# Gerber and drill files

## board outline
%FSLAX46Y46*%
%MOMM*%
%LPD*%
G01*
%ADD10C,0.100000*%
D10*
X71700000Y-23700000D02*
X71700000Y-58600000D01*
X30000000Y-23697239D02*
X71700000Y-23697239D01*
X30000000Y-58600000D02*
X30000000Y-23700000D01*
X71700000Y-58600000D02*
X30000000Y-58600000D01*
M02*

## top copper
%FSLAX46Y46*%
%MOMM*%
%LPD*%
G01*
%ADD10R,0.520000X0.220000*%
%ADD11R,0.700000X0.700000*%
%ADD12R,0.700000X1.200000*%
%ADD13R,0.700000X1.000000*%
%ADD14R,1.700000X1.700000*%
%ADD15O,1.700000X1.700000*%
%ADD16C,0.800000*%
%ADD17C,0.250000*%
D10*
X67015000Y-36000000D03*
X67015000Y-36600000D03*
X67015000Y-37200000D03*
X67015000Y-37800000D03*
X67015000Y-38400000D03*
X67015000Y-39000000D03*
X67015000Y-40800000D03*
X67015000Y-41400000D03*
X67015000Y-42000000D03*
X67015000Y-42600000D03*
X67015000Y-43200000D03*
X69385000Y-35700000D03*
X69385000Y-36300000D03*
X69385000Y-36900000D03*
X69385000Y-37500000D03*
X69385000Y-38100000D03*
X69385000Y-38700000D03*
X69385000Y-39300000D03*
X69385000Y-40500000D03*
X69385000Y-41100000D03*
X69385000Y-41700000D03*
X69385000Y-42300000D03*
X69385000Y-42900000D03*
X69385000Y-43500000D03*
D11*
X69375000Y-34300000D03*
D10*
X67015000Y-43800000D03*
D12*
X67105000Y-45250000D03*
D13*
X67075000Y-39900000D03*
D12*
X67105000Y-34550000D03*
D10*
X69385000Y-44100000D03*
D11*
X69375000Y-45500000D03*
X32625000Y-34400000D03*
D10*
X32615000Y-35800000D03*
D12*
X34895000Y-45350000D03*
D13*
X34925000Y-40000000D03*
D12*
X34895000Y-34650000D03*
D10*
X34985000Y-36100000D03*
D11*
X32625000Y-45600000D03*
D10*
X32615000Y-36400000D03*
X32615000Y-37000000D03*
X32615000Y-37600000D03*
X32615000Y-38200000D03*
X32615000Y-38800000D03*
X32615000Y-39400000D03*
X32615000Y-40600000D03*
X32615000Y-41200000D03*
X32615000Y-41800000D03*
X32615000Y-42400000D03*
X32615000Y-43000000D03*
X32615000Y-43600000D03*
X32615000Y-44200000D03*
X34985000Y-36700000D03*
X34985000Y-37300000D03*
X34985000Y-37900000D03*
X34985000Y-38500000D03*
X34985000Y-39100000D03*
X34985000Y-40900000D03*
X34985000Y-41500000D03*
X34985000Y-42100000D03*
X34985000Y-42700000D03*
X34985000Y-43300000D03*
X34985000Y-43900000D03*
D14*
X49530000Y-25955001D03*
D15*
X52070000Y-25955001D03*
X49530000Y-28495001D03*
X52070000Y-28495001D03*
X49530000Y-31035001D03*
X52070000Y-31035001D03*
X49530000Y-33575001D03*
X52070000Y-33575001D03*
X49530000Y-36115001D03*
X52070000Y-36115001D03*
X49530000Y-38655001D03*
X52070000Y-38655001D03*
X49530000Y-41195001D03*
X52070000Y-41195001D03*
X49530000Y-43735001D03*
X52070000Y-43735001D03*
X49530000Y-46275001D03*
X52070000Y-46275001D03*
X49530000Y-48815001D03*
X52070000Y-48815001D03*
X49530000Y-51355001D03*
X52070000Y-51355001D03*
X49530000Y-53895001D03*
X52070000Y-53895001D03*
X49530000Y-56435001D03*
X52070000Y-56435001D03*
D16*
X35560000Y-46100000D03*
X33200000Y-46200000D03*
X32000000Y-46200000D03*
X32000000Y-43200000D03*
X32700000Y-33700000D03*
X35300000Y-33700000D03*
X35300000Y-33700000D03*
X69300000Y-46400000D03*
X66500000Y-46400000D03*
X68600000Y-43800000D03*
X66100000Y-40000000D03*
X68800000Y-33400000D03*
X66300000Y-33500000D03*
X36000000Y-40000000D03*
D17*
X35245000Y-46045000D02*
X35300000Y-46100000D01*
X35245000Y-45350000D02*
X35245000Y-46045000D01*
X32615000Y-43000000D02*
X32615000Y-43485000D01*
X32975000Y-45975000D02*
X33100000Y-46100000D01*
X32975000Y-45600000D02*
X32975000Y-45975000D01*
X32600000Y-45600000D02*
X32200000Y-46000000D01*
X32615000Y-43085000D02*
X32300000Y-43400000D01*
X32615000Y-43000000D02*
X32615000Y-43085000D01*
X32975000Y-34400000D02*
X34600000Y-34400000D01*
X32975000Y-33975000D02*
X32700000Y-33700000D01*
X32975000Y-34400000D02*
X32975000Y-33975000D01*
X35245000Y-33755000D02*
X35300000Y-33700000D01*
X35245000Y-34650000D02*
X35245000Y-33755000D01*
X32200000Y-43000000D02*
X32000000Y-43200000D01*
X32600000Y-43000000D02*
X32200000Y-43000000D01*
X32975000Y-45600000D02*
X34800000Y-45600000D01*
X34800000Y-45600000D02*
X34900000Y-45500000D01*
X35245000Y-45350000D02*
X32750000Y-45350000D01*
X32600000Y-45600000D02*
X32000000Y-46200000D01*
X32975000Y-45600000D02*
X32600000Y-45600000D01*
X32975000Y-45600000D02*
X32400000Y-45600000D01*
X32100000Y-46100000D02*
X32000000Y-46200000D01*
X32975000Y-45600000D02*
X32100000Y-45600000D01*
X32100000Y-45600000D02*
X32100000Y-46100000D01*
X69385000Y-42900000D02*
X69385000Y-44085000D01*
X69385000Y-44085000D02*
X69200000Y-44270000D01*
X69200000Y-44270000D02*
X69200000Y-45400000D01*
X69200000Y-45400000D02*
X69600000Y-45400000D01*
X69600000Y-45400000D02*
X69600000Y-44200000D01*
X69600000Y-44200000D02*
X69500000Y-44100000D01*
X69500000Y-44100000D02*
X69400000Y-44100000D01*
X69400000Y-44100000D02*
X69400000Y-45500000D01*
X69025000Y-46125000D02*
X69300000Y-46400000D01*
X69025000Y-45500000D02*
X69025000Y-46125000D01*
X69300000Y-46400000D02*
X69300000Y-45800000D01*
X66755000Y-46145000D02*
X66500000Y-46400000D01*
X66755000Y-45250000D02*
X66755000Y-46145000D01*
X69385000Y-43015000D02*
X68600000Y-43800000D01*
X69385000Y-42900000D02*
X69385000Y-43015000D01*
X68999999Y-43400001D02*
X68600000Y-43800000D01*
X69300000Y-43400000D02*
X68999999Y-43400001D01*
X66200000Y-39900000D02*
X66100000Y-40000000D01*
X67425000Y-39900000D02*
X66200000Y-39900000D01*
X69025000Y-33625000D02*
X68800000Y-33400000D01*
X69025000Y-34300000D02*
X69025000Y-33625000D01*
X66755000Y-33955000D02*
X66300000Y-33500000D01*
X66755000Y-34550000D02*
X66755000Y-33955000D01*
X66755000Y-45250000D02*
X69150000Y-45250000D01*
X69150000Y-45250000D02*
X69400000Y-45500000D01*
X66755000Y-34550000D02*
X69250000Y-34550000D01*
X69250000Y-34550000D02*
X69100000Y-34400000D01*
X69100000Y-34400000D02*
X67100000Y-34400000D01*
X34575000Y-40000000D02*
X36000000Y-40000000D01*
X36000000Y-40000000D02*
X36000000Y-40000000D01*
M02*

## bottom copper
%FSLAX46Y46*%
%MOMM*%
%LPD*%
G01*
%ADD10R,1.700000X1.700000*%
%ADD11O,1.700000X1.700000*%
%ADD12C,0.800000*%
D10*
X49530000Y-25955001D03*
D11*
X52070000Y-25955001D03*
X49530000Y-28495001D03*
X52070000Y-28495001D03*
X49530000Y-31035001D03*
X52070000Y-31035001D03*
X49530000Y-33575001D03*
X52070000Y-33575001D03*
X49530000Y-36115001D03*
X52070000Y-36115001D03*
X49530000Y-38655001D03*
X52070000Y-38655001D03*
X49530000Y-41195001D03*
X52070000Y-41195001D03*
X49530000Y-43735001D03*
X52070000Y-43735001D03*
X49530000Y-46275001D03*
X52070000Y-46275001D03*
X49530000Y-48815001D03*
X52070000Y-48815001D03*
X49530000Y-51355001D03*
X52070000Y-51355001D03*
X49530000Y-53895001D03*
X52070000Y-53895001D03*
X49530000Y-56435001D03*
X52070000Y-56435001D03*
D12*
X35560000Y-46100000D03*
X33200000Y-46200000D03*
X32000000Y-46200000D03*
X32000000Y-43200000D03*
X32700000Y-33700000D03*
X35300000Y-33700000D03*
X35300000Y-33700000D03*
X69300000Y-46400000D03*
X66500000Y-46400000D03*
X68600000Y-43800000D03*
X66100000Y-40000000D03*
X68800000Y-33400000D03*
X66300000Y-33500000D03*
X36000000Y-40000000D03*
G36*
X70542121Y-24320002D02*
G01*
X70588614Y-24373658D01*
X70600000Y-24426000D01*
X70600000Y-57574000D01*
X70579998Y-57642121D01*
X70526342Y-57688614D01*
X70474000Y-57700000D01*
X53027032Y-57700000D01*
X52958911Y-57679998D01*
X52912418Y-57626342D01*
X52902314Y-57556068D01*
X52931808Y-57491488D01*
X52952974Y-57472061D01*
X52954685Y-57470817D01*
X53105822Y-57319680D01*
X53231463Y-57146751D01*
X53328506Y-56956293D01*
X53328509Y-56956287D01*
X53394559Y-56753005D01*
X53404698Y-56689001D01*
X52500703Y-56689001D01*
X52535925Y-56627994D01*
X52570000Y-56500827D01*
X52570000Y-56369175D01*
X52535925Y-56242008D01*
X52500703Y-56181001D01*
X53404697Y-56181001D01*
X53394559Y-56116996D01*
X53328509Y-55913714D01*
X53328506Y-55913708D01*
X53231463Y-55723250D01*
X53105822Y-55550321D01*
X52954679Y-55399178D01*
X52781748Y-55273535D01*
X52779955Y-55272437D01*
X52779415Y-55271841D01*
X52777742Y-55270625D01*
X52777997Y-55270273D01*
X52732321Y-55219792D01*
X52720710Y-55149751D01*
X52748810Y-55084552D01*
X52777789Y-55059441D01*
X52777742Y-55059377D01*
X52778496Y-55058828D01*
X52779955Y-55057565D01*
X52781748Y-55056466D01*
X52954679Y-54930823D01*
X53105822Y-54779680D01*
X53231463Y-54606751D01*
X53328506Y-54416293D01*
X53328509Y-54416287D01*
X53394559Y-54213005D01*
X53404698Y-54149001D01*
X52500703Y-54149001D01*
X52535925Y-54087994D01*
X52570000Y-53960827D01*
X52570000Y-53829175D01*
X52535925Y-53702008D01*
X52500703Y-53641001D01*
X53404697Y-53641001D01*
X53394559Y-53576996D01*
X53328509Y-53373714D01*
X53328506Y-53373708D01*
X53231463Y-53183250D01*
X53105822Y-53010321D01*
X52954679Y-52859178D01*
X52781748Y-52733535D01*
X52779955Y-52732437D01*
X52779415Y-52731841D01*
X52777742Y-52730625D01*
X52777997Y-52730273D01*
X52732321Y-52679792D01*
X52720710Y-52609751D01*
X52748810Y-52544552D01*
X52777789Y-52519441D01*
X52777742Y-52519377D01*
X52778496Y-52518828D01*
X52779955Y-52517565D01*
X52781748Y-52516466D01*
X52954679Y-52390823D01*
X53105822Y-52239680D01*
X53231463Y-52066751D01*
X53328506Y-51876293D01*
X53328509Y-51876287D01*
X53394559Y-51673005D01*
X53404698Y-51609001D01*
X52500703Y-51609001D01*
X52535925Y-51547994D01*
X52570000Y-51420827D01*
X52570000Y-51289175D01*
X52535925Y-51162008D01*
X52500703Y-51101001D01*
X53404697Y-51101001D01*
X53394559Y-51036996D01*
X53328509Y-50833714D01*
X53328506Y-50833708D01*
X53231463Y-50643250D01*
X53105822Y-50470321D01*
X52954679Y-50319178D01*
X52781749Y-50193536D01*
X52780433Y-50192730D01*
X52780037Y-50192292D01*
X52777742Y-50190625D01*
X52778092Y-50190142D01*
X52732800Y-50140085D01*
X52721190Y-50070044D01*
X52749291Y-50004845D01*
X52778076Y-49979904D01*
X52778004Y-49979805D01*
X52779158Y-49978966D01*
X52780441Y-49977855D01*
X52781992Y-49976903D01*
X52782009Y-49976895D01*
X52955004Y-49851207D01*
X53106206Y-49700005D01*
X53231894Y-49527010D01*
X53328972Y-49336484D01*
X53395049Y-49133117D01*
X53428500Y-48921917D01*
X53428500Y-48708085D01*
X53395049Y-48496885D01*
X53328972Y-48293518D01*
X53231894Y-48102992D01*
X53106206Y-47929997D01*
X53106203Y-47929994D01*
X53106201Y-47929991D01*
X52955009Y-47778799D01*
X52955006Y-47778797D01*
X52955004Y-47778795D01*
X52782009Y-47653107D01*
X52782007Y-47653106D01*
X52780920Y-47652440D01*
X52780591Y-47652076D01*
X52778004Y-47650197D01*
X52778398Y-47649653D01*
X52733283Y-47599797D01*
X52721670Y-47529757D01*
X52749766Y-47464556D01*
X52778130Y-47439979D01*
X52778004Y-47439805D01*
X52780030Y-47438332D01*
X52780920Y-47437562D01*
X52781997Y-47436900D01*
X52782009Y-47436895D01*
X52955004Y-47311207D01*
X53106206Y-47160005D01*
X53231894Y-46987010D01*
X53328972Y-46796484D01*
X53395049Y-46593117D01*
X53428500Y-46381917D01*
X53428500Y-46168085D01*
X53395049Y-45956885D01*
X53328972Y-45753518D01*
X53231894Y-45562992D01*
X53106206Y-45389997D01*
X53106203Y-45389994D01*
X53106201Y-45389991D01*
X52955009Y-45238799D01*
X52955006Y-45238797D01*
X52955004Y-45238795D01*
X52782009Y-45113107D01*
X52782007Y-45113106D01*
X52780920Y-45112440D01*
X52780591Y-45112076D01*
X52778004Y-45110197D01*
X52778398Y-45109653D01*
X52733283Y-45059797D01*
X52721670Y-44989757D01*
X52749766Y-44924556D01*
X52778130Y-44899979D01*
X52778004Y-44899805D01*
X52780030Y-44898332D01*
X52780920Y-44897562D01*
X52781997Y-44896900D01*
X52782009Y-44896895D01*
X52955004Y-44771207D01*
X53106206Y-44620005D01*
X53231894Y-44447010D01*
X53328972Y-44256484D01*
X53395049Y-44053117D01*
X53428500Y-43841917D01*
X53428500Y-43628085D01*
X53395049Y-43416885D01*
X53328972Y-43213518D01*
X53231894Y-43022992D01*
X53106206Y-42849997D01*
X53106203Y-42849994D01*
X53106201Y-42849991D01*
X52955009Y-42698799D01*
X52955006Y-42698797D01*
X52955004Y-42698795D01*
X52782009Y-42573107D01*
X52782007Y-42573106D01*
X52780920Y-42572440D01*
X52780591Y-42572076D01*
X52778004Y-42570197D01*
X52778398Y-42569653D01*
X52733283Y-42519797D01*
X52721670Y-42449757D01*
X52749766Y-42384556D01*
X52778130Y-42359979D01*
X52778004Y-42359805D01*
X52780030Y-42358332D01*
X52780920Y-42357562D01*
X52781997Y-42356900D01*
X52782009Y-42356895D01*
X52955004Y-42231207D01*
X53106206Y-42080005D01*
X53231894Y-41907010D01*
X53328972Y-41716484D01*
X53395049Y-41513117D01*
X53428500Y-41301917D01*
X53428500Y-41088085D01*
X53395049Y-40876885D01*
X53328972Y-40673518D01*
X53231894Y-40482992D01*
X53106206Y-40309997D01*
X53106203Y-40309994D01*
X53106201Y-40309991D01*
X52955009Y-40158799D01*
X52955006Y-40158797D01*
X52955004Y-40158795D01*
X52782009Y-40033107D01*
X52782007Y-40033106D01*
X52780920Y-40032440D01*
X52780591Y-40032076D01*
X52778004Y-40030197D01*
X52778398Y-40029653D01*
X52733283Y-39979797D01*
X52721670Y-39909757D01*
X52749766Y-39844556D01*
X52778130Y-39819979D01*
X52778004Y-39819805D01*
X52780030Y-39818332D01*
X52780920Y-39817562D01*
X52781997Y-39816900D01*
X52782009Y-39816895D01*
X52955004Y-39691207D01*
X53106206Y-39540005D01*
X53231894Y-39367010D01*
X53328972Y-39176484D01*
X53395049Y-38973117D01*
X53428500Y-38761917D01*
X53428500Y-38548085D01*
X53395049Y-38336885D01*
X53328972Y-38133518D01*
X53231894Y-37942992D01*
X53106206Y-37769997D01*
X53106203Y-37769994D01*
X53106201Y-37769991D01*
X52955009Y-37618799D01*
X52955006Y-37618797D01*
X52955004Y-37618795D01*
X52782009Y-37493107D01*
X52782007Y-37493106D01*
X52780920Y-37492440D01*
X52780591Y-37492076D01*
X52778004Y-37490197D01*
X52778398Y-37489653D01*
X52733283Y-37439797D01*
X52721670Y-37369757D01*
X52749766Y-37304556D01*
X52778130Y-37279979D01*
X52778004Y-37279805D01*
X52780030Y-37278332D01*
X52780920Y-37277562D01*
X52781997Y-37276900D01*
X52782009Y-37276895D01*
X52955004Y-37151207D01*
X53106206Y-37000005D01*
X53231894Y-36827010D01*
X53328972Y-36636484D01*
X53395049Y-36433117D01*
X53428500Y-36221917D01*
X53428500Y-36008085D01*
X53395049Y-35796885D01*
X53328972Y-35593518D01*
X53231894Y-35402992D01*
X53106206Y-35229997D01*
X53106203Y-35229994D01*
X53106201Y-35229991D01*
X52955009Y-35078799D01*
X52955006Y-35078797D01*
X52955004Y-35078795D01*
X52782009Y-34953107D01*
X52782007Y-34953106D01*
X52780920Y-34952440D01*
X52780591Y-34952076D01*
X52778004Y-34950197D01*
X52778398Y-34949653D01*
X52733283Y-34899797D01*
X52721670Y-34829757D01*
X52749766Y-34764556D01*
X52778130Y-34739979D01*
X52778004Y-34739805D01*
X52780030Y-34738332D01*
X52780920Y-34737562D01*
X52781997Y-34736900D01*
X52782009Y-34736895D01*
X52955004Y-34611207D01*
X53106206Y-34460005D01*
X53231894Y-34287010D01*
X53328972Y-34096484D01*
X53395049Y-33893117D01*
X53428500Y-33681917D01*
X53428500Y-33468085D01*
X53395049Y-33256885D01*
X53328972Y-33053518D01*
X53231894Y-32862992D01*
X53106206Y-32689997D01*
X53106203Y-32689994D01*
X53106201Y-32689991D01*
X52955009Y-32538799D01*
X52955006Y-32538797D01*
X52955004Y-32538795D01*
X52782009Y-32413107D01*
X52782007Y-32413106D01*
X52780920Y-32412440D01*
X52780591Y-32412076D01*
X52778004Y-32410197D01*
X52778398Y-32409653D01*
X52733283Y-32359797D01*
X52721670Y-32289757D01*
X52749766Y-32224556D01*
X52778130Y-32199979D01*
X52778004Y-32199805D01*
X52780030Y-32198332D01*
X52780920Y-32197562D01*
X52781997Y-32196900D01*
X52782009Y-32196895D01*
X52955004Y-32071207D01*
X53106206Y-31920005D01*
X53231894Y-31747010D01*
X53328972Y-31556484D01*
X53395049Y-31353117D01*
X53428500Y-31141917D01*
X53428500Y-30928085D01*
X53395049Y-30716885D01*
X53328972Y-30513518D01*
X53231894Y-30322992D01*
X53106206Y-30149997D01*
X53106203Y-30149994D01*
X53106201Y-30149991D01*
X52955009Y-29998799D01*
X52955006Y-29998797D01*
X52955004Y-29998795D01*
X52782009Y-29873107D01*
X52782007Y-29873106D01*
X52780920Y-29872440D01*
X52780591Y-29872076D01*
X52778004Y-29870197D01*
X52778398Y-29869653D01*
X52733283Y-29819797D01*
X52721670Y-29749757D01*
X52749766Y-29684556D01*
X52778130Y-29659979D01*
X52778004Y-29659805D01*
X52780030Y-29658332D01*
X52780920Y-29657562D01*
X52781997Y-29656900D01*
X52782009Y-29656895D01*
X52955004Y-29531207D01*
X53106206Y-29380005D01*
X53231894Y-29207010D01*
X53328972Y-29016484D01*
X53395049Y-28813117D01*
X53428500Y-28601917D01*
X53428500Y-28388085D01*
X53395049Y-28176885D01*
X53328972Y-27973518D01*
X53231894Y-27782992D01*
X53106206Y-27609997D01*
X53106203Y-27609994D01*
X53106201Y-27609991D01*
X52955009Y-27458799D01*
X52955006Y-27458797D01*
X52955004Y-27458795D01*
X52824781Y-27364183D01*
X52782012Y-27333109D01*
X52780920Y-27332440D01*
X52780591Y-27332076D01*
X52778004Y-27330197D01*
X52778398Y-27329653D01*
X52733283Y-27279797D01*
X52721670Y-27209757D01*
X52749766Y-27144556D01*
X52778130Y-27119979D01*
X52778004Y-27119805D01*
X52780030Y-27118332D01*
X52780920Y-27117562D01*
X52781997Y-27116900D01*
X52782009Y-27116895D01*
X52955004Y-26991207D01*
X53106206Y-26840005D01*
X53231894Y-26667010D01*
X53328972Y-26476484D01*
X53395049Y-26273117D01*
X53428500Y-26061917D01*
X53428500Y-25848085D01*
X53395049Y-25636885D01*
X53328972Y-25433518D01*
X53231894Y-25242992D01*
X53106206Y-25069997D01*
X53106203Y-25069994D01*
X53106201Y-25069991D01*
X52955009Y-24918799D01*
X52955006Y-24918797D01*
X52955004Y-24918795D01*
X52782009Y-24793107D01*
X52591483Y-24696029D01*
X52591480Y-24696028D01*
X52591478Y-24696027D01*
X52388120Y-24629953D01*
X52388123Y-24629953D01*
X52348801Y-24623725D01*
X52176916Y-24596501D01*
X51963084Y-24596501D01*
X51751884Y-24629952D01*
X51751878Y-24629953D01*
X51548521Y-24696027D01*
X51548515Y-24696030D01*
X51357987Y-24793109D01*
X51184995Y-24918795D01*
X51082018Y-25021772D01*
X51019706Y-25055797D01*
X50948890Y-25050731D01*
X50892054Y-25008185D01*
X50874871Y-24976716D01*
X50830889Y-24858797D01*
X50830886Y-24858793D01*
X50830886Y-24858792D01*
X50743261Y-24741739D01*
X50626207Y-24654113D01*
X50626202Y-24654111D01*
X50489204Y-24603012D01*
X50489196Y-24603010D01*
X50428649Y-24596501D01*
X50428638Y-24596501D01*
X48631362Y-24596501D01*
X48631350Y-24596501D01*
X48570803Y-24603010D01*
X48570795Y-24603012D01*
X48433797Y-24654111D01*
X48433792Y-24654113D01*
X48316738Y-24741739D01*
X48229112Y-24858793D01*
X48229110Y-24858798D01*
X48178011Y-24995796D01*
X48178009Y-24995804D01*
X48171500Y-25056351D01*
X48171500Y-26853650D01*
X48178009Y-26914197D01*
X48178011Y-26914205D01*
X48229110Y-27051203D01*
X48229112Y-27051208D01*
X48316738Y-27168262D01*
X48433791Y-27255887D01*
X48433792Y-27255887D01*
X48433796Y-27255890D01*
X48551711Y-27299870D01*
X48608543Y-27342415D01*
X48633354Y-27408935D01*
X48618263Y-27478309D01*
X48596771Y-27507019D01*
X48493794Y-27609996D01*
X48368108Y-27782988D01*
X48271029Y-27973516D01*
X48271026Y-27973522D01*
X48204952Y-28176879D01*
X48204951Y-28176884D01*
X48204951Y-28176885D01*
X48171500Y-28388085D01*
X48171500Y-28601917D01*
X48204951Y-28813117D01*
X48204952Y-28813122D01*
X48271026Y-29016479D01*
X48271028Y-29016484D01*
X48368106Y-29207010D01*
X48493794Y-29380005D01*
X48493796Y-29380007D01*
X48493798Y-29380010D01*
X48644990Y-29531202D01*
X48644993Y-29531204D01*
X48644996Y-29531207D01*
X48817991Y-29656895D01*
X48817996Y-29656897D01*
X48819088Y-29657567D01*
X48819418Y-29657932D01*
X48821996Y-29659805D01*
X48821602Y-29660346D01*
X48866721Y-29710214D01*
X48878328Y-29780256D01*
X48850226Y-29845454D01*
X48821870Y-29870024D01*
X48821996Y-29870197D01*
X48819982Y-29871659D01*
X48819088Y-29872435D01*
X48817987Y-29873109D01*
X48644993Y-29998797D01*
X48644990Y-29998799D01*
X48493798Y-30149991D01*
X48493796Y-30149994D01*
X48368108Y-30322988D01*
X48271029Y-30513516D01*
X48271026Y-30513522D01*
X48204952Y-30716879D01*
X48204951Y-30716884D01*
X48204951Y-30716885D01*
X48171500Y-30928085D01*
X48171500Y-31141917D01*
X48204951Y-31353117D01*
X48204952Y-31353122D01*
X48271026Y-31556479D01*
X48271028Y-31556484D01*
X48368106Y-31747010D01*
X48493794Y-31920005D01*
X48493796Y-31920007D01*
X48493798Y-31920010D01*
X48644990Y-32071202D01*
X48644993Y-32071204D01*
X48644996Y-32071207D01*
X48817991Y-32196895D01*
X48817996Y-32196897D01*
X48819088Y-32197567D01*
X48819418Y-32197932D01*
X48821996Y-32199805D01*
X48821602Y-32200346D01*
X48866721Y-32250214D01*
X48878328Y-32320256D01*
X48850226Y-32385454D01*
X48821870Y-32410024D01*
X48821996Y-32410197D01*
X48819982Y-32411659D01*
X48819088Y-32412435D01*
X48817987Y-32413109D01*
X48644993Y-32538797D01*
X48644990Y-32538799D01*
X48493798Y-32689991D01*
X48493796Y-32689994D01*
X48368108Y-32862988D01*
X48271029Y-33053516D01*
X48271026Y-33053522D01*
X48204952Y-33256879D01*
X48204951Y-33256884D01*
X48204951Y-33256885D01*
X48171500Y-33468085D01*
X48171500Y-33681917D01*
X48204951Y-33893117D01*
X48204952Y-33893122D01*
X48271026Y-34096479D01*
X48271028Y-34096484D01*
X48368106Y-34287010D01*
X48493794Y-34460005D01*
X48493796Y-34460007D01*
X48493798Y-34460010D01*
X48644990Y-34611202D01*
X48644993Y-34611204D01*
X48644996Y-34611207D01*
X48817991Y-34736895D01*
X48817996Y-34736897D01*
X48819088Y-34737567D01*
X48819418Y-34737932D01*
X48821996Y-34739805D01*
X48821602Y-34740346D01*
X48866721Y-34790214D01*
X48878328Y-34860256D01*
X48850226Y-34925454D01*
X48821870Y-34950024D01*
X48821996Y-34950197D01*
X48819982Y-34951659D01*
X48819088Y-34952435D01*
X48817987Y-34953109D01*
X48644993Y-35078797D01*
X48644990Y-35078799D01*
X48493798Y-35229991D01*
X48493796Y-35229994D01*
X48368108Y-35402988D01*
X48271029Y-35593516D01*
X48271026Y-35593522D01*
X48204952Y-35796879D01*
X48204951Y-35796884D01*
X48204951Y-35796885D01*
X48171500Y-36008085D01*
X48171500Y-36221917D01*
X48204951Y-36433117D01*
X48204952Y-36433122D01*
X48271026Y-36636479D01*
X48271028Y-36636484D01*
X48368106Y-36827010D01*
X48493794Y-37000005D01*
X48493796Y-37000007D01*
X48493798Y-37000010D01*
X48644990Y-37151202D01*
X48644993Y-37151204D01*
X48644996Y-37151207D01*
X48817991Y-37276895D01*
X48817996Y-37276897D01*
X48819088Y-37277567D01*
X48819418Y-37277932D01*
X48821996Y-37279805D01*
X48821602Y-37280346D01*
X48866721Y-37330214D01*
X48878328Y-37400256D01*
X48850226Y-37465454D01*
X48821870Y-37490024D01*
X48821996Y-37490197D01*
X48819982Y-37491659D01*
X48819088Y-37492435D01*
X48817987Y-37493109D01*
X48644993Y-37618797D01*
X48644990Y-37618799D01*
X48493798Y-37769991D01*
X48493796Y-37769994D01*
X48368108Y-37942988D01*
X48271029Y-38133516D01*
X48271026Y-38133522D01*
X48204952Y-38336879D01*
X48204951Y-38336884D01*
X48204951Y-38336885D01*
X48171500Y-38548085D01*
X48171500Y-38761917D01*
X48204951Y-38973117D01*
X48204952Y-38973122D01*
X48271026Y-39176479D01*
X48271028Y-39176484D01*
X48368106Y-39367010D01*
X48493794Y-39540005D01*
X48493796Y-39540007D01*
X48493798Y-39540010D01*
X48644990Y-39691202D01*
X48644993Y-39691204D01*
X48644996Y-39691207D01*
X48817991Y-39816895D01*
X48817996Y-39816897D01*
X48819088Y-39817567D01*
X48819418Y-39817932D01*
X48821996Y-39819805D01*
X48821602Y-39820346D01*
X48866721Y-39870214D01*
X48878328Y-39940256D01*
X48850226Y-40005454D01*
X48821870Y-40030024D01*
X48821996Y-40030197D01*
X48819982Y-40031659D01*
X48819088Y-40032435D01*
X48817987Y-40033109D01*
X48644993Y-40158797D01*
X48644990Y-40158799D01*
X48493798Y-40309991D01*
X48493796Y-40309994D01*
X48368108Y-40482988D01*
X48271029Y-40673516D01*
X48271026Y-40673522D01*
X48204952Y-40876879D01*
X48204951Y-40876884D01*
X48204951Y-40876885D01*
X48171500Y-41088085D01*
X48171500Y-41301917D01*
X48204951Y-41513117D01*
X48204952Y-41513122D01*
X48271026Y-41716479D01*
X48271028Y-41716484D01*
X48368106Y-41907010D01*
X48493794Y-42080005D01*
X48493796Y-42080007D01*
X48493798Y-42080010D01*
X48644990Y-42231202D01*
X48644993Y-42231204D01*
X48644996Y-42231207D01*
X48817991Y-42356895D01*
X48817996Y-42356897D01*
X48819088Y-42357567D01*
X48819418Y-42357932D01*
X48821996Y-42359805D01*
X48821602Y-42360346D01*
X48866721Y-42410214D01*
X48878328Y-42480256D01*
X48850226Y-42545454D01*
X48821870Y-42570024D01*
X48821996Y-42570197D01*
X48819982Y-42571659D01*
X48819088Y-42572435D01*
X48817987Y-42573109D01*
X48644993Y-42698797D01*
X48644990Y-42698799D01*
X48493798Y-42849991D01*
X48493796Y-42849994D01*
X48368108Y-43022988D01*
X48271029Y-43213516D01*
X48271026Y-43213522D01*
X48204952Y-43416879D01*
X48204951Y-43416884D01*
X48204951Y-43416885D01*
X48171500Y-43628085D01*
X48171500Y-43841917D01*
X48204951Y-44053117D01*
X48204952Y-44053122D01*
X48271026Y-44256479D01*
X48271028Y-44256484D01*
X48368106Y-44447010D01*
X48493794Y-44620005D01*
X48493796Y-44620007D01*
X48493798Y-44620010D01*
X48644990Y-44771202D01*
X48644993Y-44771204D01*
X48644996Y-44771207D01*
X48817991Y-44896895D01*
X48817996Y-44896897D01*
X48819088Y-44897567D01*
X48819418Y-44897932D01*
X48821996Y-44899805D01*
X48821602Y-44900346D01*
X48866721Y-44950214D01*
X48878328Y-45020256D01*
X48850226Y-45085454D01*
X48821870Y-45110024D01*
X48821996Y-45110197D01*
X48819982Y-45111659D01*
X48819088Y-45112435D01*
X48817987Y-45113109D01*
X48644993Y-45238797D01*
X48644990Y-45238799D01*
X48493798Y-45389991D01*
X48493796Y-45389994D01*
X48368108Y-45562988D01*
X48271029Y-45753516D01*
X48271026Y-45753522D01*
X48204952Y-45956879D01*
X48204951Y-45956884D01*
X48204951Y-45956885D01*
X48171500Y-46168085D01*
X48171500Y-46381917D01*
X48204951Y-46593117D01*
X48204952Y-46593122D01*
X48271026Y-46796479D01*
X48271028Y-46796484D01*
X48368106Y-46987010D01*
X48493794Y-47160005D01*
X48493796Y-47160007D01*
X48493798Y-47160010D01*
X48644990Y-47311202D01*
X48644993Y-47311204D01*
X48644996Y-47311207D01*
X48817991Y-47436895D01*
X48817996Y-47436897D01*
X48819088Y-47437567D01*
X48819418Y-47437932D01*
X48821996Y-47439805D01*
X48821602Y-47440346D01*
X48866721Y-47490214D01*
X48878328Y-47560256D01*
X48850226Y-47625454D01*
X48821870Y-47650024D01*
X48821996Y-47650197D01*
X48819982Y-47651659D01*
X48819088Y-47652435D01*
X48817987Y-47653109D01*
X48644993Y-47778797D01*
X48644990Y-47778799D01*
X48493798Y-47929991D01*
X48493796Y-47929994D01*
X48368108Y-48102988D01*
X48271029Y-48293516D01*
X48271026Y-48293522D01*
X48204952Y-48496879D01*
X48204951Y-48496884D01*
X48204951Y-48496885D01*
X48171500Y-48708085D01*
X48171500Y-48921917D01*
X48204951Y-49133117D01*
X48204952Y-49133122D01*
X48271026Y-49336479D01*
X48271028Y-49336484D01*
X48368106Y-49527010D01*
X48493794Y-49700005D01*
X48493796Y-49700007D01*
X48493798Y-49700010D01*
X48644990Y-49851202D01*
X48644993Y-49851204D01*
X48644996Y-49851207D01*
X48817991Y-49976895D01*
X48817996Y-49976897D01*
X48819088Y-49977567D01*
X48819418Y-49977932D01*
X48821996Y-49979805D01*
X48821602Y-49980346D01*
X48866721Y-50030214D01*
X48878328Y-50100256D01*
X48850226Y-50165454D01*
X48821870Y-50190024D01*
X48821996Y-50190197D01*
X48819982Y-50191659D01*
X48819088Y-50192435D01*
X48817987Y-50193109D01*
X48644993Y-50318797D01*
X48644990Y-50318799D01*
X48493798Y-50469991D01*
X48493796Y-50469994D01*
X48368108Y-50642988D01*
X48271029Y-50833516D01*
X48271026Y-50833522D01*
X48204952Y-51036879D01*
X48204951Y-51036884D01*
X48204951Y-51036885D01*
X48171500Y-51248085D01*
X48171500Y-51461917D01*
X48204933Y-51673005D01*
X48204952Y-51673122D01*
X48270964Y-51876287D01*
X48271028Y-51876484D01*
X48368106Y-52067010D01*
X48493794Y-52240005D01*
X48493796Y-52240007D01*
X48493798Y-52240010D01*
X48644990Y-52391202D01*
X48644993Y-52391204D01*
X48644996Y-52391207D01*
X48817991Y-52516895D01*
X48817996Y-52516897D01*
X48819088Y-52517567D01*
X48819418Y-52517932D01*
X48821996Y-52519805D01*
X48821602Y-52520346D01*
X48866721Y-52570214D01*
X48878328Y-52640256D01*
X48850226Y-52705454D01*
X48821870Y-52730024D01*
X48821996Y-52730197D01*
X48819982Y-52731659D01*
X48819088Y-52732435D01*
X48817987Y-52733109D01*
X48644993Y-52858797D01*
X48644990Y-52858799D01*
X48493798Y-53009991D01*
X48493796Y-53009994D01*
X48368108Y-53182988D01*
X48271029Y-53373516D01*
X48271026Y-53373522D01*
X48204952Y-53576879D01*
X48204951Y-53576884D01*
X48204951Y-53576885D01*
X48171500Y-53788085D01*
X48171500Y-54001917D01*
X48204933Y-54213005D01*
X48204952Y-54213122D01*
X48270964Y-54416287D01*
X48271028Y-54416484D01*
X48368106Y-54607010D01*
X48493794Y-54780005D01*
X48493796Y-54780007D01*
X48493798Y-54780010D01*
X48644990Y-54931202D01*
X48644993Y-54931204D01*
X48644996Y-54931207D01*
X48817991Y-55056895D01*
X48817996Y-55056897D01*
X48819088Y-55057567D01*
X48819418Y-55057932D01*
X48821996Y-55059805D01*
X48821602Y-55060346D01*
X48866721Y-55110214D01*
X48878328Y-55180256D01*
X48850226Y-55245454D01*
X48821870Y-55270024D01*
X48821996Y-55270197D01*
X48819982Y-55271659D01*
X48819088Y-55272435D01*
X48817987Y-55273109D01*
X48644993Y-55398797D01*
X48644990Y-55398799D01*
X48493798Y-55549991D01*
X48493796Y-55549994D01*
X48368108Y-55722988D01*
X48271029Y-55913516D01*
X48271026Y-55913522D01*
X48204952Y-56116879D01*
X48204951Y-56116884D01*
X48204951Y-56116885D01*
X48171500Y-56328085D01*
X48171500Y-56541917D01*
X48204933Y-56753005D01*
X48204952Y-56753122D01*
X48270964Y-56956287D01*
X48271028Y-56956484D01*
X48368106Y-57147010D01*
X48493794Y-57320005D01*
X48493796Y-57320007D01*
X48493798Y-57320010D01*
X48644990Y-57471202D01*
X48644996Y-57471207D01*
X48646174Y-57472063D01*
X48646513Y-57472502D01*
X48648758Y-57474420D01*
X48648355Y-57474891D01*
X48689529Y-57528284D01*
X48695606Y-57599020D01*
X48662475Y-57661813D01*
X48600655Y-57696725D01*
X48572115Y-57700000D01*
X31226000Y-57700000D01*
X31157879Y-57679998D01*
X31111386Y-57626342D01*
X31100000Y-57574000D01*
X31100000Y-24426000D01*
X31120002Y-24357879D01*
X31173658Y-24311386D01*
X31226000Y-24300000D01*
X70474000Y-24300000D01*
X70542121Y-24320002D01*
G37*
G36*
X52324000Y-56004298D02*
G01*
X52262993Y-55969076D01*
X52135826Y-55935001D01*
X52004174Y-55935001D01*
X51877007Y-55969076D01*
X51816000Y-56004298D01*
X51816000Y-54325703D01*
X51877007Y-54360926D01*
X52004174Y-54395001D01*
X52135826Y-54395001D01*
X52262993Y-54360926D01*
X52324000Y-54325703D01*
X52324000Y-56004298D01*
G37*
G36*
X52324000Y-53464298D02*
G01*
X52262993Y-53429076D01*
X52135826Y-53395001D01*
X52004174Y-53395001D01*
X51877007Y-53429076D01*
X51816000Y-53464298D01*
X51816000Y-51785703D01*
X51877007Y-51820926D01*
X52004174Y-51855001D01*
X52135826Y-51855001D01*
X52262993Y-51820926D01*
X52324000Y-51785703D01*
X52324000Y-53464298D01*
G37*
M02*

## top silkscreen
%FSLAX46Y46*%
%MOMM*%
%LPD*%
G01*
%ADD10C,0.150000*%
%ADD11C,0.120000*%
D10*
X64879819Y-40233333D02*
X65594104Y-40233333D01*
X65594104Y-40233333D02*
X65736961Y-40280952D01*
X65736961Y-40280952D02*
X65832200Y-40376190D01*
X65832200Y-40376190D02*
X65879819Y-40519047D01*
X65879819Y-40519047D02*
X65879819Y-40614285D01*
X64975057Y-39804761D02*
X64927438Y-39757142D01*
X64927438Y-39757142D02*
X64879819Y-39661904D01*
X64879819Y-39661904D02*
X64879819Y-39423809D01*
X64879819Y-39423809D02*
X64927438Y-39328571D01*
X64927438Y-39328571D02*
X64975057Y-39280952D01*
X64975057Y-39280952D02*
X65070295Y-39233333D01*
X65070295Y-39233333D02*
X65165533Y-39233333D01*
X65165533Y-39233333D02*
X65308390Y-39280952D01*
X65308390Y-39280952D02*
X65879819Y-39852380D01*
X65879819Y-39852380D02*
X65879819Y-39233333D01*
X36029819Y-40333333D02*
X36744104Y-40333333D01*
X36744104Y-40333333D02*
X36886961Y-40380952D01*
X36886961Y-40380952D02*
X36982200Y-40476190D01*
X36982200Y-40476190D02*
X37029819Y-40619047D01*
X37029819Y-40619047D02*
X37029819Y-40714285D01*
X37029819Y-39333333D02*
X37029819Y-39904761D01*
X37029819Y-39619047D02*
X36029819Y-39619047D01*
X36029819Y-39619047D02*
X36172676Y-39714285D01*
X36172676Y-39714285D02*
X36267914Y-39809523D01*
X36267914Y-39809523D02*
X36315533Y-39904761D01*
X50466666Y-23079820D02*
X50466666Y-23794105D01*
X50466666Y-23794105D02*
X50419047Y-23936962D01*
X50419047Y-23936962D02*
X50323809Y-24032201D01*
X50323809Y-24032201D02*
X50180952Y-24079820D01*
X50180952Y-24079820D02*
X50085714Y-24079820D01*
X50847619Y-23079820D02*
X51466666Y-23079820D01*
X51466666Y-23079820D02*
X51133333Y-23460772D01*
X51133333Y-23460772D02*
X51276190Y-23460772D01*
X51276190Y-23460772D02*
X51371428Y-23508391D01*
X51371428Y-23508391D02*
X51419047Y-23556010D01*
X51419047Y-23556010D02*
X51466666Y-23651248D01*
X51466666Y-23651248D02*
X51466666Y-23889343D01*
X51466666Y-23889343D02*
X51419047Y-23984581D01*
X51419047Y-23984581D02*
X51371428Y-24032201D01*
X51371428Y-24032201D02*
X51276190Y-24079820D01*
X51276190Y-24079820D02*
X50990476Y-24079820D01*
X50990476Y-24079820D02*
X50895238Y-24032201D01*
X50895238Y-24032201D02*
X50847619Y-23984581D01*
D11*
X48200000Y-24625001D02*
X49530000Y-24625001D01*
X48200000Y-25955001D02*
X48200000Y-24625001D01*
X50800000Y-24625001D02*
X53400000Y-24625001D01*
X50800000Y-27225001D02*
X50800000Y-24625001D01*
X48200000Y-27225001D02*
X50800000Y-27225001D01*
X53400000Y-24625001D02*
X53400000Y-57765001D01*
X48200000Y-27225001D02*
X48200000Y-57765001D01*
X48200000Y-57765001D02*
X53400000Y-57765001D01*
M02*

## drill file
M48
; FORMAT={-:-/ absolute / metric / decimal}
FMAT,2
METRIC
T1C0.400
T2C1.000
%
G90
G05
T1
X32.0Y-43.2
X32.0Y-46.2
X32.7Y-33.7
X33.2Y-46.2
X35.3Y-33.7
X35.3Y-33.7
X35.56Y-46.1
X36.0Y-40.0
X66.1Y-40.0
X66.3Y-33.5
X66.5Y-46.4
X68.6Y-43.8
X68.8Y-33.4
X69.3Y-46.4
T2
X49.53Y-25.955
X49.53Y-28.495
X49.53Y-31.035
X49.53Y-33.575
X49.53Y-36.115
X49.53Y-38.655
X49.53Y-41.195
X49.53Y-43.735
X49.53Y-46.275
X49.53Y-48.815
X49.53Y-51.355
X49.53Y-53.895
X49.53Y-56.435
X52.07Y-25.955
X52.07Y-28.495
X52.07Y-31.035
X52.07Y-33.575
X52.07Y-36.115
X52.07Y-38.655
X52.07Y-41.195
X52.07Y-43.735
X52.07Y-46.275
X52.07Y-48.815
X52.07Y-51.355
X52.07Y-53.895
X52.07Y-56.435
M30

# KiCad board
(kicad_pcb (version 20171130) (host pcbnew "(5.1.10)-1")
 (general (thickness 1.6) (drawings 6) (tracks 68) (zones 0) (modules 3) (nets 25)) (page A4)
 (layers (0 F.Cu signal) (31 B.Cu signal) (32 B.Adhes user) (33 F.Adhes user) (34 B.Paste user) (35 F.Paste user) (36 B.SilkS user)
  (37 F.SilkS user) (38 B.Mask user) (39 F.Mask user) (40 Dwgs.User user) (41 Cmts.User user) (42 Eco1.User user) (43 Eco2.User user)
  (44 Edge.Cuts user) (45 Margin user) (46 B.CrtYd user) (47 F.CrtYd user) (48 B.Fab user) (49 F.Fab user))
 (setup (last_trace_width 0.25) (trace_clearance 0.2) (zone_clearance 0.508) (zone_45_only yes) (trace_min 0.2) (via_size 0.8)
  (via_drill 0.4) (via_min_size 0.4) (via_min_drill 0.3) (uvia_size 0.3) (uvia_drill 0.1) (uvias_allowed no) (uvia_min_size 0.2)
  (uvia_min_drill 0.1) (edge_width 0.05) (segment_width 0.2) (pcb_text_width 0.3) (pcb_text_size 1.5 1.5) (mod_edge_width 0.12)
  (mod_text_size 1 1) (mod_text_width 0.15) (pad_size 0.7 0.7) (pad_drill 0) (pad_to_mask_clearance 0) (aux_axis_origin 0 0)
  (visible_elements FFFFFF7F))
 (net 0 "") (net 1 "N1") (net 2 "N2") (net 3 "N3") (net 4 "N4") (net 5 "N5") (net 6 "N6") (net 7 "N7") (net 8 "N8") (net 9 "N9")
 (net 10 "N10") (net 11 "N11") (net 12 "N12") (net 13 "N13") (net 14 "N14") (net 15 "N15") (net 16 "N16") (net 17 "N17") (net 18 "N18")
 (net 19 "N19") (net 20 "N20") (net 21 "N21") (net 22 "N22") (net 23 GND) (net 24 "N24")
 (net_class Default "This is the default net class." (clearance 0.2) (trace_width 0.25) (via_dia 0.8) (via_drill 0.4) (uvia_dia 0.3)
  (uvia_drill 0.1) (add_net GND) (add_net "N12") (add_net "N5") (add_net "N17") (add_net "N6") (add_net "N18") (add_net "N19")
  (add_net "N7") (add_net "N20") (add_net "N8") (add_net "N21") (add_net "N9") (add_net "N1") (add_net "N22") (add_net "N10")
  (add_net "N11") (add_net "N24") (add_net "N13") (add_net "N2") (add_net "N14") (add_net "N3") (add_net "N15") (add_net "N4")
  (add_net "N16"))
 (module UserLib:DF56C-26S (layer F.Cu) (at 68.2 39.9 90)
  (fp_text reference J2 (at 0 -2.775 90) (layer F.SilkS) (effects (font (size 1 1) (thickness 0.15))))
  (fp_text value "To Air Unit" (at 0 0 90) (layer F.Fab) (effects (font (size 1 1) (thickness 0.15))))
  (pad 25 smd rect (at 3.9 -1.185 90) (size 0.22 0.52) (layers F.Cu F.Paste F.Mask) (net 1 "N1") (clearance 0.1))
  (pad 23 smd rect (at 3.3 -1.185 90) (size 0.22 0.52) (layers F.Cu F.Paste F.Mask) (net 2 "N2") (clearance 0.1))
  (pad 21 smd rect (at 2.7 -1.185 90) (size 0.22 0.52) (layers F.Cu F.Paste F.Mask) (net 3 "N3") (clearance 0.1))
  (pad 19 smd rect (at 2.1 -1.185 90) (size 0.22 0.52) (layers F.Cu F.Paste F.Mask) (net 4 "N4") (clearance 0.1))
  (pad 17 smd rect (at 1.5 -1.185 90) (size 0.22 0.52) (layers F.Cu F.Paste F.Mask) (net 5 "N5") (clearance 0.1))
  (pad 15 smd rect (at 0.9 -1.185 90) (size 0.22 0.52) (layers F.Cu F.Paste F.Mask) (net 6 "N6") (clearance 0.1))
  (pad 12 smd rect (at -0.9 -1.185 90) (size 0.22 0.52) (layers F.Cu F.Paste F.Mask) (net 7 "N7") (clearance 0.1))
  (pad 10 smd rect (at -1.5 -1.185 90) (size 0.22 0.52) (layers F.Cu F.Paste F.Mask) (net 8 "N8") (clearance 0.1))
  (pad 8 smd rect (at -2.1 -1.185 90) (size 0.22 0.52) (layers F.Cu F.Paste F.Mask) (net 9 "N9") (clearance 0.1))
  (pad 6 smd rect (at -2.7 -1.185 90) (size 0.22 0.52) (layers F.Cu F.Paste F.Mask) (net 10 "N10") (clearance 0.1))
  (pad 4 smd rect (at -3.3 -1.185 90) (size 0.22 0.52) (layers F.Cu F.Paste F.Mask) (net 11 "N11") (clearance 0.1))
  (pad 26 smd rect (at 4.2 1.185 90) (size 0.22 0.52) (layers F.Cu F.Paste F.Mask) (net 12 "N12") (clearance 0.1))
  (pad 24 smd rect (at 3.6 1.185 90) (size 0.22 0.52) (layers F.Cu F.Paste F.Mask) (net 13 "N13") (clearance 0.1))
  (pad 22 smd rect (at 3 1.185 90) (size 0.22 0.52) (layers F.Cu F.Paste F.Mask) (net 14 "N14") (clearance 0.1))
  (pad 20 smd rect (at 2.4 1.185 90) (size 0.22 0.52) (layers F.Cu F.Paste F.Mask) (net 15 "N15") (clearance 0.1))
  (pad 18 smd rect (at 1.8 1.185 90) (size 0.22 0.52) (layers F.Cu F.Paste F.Mask) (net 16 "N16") (clearance 0.1))
  (pad 16 smd rect (at 1.2 1.185 90) (size 0.22 0.52) (layers F.Cu F.Paste F.Mask) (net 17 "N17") (clearance 0.1))
  (pad 14 smd rect (at 0.6 1.185 90) (size 0.22 0.52) (layers F.Cu F.Paste F.Mask) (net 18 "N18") (clearance 0.1))
  (pad 13 smd rect (at -0.6 1.185 90) (size 0.22 0.52) (layers F.Cu F.Paste F.Mask) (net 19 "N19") (clearance 0.1))
  (pad 11 smd rect (at -1.2 1.185 90) (size 0.22 0.52) (layers F.Cu F.Paste F.Mask) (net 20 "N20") (clearance 0.1))
  (pad 9 smd rect (at -1.8 1.185 90) (size 0.22 0.52) (layers F.Cu F.Paste F.Mask) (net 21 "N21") (clearance 0.1))
  (pad 7 smd rect (at -2.4 1.185 90) (size 0.22 0.52) (layers F.Cu F.Paste F.Mask) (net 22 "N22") (clearance 0.1))
  (pad 5 smd rect (at -3 1.185 90) (size 0.22 0.52) (layers F.Cu F.Paste F.Mask) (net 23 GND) (clearance 0.1))
  (pad 3 smd rect (at -3.6 1.185 90) (size 0.22 0.52) (layers F.Cu F.Paste F.Mask) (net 23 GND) (clearance 0.1))
  (pad GND smd rect (at 5.6 0.825 90) (size 0.7 0.7) (drill (offset 0 0.35)) (layers F.Cu F.Paste F.Mask) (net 23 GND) (clearance 0.1))
  (pad 2 smd rect (at -3.9 -1.185 90) (size 0.22 0.52) (layers F.Cu F.Paste F.Mask) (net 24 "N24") (clearance 0.1))
  (pad GND smd rect (at -5.35 -1.445 90) (size 1.2 0.7) (drill (offset 0 0.35)) (layers F.Cu F.Paste F.Mask) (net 23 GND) (clearance 0.1))
  (pad GND smd rect (at 0 -0.775 90) (size 1 0.7) (drill (offset 0 -0.35)) (layers F.Cu F.Paste F.Mask) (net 23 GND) (clearance 0.1))
  (pad GND smd rect (at 5.35 -1.445 90) (size 1.2 0.7) (drill (offset 0 0.35)) (layers F.Cu F.Paste F.Mask) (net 23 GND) (clearance 0.1))
  (pad 1 smd rect (at -4.2 1.185 90) (size 0.22 0.52) (layers F.Cu F.Paste F.Mask) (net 23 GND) (clearance 0.1))
  (pad GND smd rect (at -5.6 0.825 90) (size 0.7 0.7) (drill (offset 0 0.35)) (layers F.Cu F.Paste F.Mask) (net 23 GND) (clearance 0.1)))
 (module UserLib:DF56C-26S (layer F.Cu) (at 33.8 40 270)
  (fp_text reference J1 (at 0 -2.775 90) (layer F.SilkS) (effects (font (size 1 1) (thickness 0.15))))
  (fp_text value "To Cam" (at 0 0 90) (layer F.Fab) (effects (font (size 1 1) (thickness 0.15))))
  (pad GND smd rect (at -5.6 0.825 270) (size 0.7 0.7) (drill (offset 0 0.35)) (layers F.Cu F.Paste F.Mask) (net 23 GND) (clearance 0.1))
  (pad 1 smd rect (at -4.2 1.185 270) (size 0.22 0.52) (layers F.Cu F.Paste F.Mask) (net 12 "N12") (clearance 0.1))
  (pad GND smd rect (at 5.35 -1.445 270) (size 1.2 0.7) (drill (offset 0 0.35)) (layers F.Cu F.Paste F.Mask) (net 23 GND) (clearance 0.1))
  (pad GND smd rect (at 0 -0.775 270) (size 1 0.7) (drill (offset 0 -0.35)) (layers F.Cu F.Paste F.Mask) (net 23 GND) (clearance 0.1))
  (pad GND smd rect (at -5.35 -1.445 270) (size 1.2 0.7) (drill (offset 0 0.35)) (layers F.Cu F.Paste F.Mask) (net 23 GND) (clearance 0.1))
  (pad 2 smd rect (at -3.9 -1.185 270) (size 0.22 0.52) (layers F.Cu F.Paste F.Mask) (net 1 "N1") (clearance 0.1))
  (pad GND smd rect (at 5.6 0.825 270) (size 0.7 0.7) (drill (offset 0 0.35)) (layers F.Cu F.Paste F.Mask) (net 23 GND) (clearance 0.1))
  (pad 3 smd rect (at -3.6 1.185 270) (size 0.22 0.52) (layers F.Cu F.Paste F.Mask) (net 13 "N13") (clearance 0.1))
  (pad 5 smd rect (at -3 1.185 270) (size 0.22 0.52) (layers F.Cu F.Paste F.Mask) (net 14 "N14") (clearance 0.1))
  (pad 7 smd rect (at -2.4 1.185 270) (size 0.22 0.52) (layers F.Cu F.Paste F.Mask) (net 15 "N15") (clearance 0.1))
  (pad 9 smd rect (at -1.8 1.185 270) (size 0.22 0.52) (layers F.Cu F.Paste F.Mask) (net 16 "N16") (clearance 0.1))
  (pad 11 smd rect (at -1.2 1.185 270) (size 0.22 0.52) (layers F.Cu F.Paste F.Mask) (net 17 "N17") (clearance 0.1))
  (pad 13 smd rect (at -0.6 1.185 270) (size 0.22 0.52) (layers F.Cu F.Paste F.Mask) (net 18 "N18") (clearance 0.1))
  (pad 14 smd rect (at 0.6 1.185 270) (size 0.22 0.52) (layers F.Cu F.Paste F.Mask) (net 19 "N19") (clearance 0.1))
  (pad 16 smd rect (at 1.2 1.185 270) (size 0.22 0.52) (layers F.Cu F.Paste F.Mask) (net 20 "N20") (clearance 0.1))
  (pad 18 smd rect (at 1.8 1.185 270) (size 0.22 0.52) (layers F.Cu F.Paste F.Mask) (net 21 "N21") (clearance 0.1))
  (pad 20 smd rect (at 2.4 1.185 270) (size 0.22 0.52) (layers F.Cu F.Paste F.Mask) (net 22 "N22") (clearance 0.1))
  (pad 22 smd rect (at 3 1.185 270) (size 0.22 0.52) (layers F.Cu F.Paste F.Mask) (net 23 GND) (clearance 0.1))
  (pad 24 smd rect (at 3.6 1.185 270) (size 0.22 0.52) (layers F.Cu F.Paste F.Mask) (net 23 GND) (clearance 0.1))
  (pad 26 smd rect (at 4.2 1.185 270) (size 0.22 0.52) (layers F.Cu F.Paste F.Mask) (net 23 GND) (clearance 0.1))
  (pad 4 smd rect (at -3.3 -1.185 270) (size 0.22 0.52) (layers F.Cu F.Paste F.Mask) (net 2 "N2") (clearance 0.1))
  (pad 6 smd rect (at -2.7 -1.185 270) (size 0.22 0.52) (layers F.Cu F.Paste F.Mask) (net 3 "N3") (clearance 0.1))
  (pad 8 smd rect (at -2.1 -1.185 270) (size 0.22 0.52) (layers F.Cu F.Paste F.Mask) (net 4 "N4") (clearance 0.1))
  (pad 10 smd rect (at -1.5 -1.185 270) (size 0.22 0.52) (layers F.Cu F.Paste F.Mask) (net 5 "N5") (clearance 0.1))
  (pad 12 smd rect (at -0.9 -1.185 270) (size 0.22 0.52) (layers F.Cu F.Paste F.Mask) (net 6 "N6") (clearance 0.1))
  (pad 15 smd rect (at 0.9 -1.185 270) (size 0.22 0.52) (layers F.Cu F.Paste F.Mask) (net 7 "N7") (clearance 0.1))
  (pad 17 smd rect (at 1.5 -1.185 270) (size 0.22 0.52) (layers F.Cu F.Paste F.Mask) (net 8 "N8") (clearance 0.1))
  (pad 19 smd rect (at 2.1 -1.185 270) (size 0.22 0.52) (layers F.Cu F.Paste F.Mask) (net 9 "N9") (clearance 0.1))
  (pad 21 smd rect (at 2.7 -1.185 270) (size 0.22 0.52) (layers F.Cu F.Paste F.Mask) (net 10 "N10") (clearance 0.1))
  (pad 23 smd rect (at 3.3 -1.185 270) (size 0.22 0.52) (layers F.Cu F.Paste F.Mask) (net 11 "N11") (clearance 0.1))
  (pad 25 smd rect (at 3.9 -1.185 270) (size 0.22 0.52) (layers F.Cu F.Paste F.Mask) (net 24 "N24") (clearance 0.1)))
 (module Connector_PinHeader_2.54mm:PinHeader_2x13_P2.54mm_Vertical (layer F.Cu) (at 49.53 25.955001)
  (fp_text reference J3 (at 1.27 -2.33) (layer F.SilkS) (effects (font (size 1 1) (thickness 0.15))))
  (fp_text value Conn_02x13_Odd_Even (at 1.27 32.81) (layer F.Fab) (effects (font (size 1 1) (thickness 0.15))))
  (fp_line (start -1.33 -1.33) (end 0 -1.33) (layer F.SilkS) (width 0.12))
  (fp_line (start -1.33 0) (end -1.33 -1.33) (layer F.SilkS) (width 0.12))
  (fp_line (start 1.27 -1.33) (end 3.87 -1.33) (layer F.SilkS) (width 0.12))
  (fp_line (start 1.27 1.27) (end 1.27 -1.33) (layer F.SilkS) (width 0.12))
  (fp_line (start -1.33 1.27) (end 1.27 1.27) (layer F.SilkS) (width 0.12))
  (fp_line (start 3.87 -1.33) (end 3.87 31.81) (layer F.SilkS) (width 0.12))
  (fp_line (start -1.33 1.27) (end -1.33 31.81) (layer F.SilkS) (width 0.12))
  (fp_line (start -1.33 31.81) (end 3.87 31.81) (layer F.SilkS) (width 0.12))
  (pad 1 thru_hole rect (at 0 0) (size 1.7 1.7) (drill 1) (layers *.Cu *.Mask) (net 12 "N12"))
  (pad 2 thru_hole oval (at 2.54 0) (size 1.7 1.7) (drill 1) (layers *.Cu *.Mask) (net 1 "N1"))
  (pad 3 thru_hole oval (at 0 2.54) (size 1.7 1.7) (drill 1) (layers *.Cu *.Mask) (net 13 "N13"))
  (pad 4 thru_hole oval (at 2.54 2.54) (size 1.7 1.7) (drill 1) (layers *.Cu *.Mask) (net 2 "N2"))
  (pad 5 thru_hole oval (at 0 5.08) (size 1.7 1.7) (drill 1) (layers *.Cu *.Mask) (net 14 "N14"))
  (pad 6 thru_hole oval (at 2.54 5.08) (size 1.7 1.7) (drill 1) (layers *.Cu *.Mask) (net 3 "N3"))
  (pad 7 thru_hole oval (at 0 7.62) (size 1.7 1.7) (drill 1) (layers *.Cu *.Mask) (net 15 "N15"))
  (pad 8 thru_hole oval (at 2.54 7.62) (size 1.7 1.7) (drill 1) (layers *.Cu *.Mask) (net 4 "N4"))
  (pad 9 thru_hole oval (at 0 10.16) (size 1.7 1.7) (drill 1) (layers *.Cu *.Mask) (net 16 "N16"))
  (pad 10 thru_hole oval (at 2.54 10.16) (size 1.7 1.7) (drill 1) (layers *.Cu *.Mask) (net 5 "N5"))
  (pad 11 thru_hole oval (at 0 12.7) (size 1.7 1.7) (drill 1) (layers *.Cu *.Mask) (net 17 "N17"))
  (pad 12 thru_hole oval (at 2.54 12.7) (size 1.7 1.7) (drill 1) (layers *.Cu *.Mask) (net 6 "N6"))
  (pad 13 thru_hole oval (at 0 15.24) (size 1.7 1.7) (drill 1) (layers *.Cu *.Mask) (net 18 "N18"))
  (pad 14 thru_hole oval (at 2.54 15.24) (size 1.7 1.7) (drill 1) (layers *.Cu *.Mask) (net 19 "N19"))
  (pad 15 thru_hole oval (at 0 17.78) (size 1.7 1.7) (drill 1) (layers *.Cu *.Mask) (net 7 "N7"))
  (pad 16 thru_hole oval (at 2.54 17.78) (size 1.7 1.7) (drill 1) (layers *.Cu *.Mask) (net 20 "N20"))
  (pad 17 thru_hole oval (at 0 20.32) (size 1.7 1.7) (drill 1) (layers *.Cu *.Mask) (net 8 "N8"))
  (pad 18 thru_hole oval (at 2.54 20.32) (size 1.7 1.7) (drill 1) (layers *.Cu *.Mask) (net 21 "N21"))
  (pad 19 thru_hole oval (at 0 22.86) (size 1.7 1.7) (drill 1) (layers *.Cu *.Mask) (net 9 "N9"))
  (pad 20 thru_hole oval (at 2.54 22.86) (size 1.7 1.7) (drill 1) (layers *.Cu *.Mask) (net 22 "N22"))
  (pad 21 thru_hole oval (at 0 25.4) (size 1.7 1.7) (drill 1) (layers *.Cu *.Mask) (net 10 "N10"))
  (pad 22 thru_hole oval (at 2.54 25.4) (size 1.7 1.7) (drill 1) (layers *.Cu *.Mask) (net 23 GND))
  (pad 23 thru_hole oval (at 0 27.94) (size 1.7 1.7) (drill 1) (layers *.Cu *.Mask) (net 11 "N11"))
  (pad 24 thru_hole oval (at 2.54 27.94) (size 1.7 1.7) (drill 1) (layers *.Cu *.Mask) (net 23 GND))
  (pad 25 thru_hole oval (at 0 30.48) (size 1.7 1.7) (drill 1) (layers *.Cu *.Mask) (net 24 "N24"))
  (pad 26 thru_hole oval (at 2.54 30.48) (size 1.7 1.7) (drill 1) (layers *.Cu *.Mask) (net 23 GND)))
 (gr_line (start 71.7 23.7) (end 71.7 58.6) (layer Edge.Cuts) (width 0.1))
 (gr_line (start 30 23.697239) (end 71.7 23.697239) (layer Edge.Cuts) (width 0.1))
 (gr_line (start 30 58.6) (end 30 23.7) (layer Edge.Cuts) (width 0.1))
 (gr_line (start 71.7 58.6) (end 30 58.6) (layer Edge.Cuts) (width 0.1))
 (via (at 35.56 46.1) (size 0.8) (drill 0.4) (layers F.Cu B.Cu) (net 23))
 (segment (start 35.245 46.045) (end 35.3 46.1) (width 0.25) (layer F.Cu) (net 23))
 (segment (start 35.245 45.35) (end 35.245 46.045) (width 0.25) (layer F.Cu) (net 23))
 (segment (start 32.615 43) (end 32.615 43.485) (width 0.25) (layer F.Cu) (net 23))
 (via (at 33.2 46.2) (size 0.8) (drill 0.4) (layers F.Cu B.Cu) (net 23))
 (segment (start 32.975 45.975) (end 33.1 46.1) (width 0.25) (layer F.Cu) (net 23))
 (segment (start 32.975 45.6) (end 32.975 45.975) (width 0.25) (layer F.Cu) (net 23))
 (via (at 32 46.2) (size 0.8) (drill 0.4) (layers F.Cu B.Cu) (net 23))
 (segment (start 32.6 45.6) (end 32.2 46) (width 0.25) (layer F.Cu) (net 23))
 (via (at 32 43.2) (size 0.8) (drill 0.4) (layers F.Cu B.Cu) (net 23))
 (segment (start 32.615 43.085) (end 32.3 43.4) (width 0.25) (layer F.Cu) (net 23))
 (segment (start 32.615 43) (end 32.615 43.085) (width 0.25) (layer F.Cu) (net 23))
 (segment (start 32.975 34.4) (end 34.6 34.4) (width 0.25) (layer F.Cu) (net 23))
 (via (at 32.7 33.7) (size 0.8) (drill 0.4) (layers F.Cu B.Cu) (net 23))
 (segment (start 32.975 33.975) (end 32.7 33.7) (width 0.25) (layer F.Cu) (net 23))
 (segment (start 32.975 34.4) (end 32.975 33.975) (width 0.25) (layer F.Cu) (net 23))
 (via (at 35.3 33.7) (size 0.8) (drill 0.4) (layers F.Cu B.Cu) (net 23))
 (segment (start 35.245 33.755) (end 35.3 33.7) (width 0.25) (layer F.Cu) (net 23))
 (segment (start 35.245 34.65) (end 35.245 33.755) (width 0.25) (layer F.Cu) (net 23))
 (via (at 35.3 33.7) (size 0.8) (drill 0.4) (layers F.Cu B.Cu) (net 23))
 (segment (start 32.2 43) (end 32 43.2) (width 0.25) (layer F.Cu) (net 23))
 (segment (start 32.6 43) (end 32.2 43) (width 0.25) (layer F.Cu) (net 23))
 (segment (start 32.975 45.6) (end 34.8 45.6) (width 0.25) (layer F.Cu) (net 23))
 (segment (start 34.8 45.6) (end 34.9 45.5) (width 0.25) (layer F.Cu) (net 23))
 (segment (start 35.245 45.35) (end 32.75 45.35) (width 0.25) (layer F.Cu) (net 23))
 (segment (start 32.6 45.6) (end 32 46.2) (width 0.25) (layer F.Cu) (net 23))
 (segment (start 32.975 45.6) (end 32.6 45.6) (width 0.25) (layer F.Cu) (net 23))
 (segment (start 32.975 45.6) (end 32.4 45.6) (width 0.25) (layer F.Cu) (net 23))
 (segment (start 32.1 46.1) (end 32 46.2) (width 0.25) (layer F.Cu) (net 23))
 (segment (start 32.975 45.6) (end 32.1 45.6) (width 0.25) (layer F.Cu) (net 23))
 (segment (start 32.1 45.6) (end 32.1 46.1) (width 0.25) (layer F.Cu) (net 23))
 (segment (start 69.385 42.9) (end 69.385 44.085) (width 0.25) (layer F.Cu) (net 23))
 (segment (start 69.385 44.085) (end 69.2 44.27) (width 0.25) (layer F.Cu) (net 23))
 (segment (start 69.2 44.27) (end 69.2 45.4) (width 0.25) (layer F.Cu) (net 23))
 (segment (start 69.2 45.4) (end 69.6 45.4) (width 0.25) (layer F.Cu) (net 23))
 (segment (start 69.6 45.4) (end 69.6 44.2) (width 0.25) (layer F.Cu) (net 23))
 (segment (start 69.6 44.2) (end 69.5 44.1) (width 0.25) (layer F.Cu) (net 23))
 (segment (start 69.5 44.1) (end 69.4 44.1) (width 0.25) (layer F.Cu) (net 23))
 (segment (start 69.4 44.1) (end 69.4 45.5) (width 0.25) (layer F.Cu) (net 23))
 (via (at 69.3 46.4) (size 0.8) (drill 0.4) (layers F.Cu B.Cu) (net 23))
 (segment (start 69.025 46.125) (end 69.3 46.4) (width 0.25) (layer F.Cu) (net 23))
 (segment (start 69.025 45.5) (end 69.025 46.125) (width 0.25) (layer F.Cu) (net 23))
 (segment (start 69.3 46.4) (end 69.3 45.8) (width 0.25) (layer F.Cu) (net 23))
 (via (at 66.5 46.4) (size 0.8) (drill 0.4) (layers F.Cu B.Cu) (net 23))
 (segment (start 66.755 46.145) (end 66.5 46.4) (width 0.25) (layer F.Cu) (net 23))
 (segment (start 66.755 45.25) (end 66.755 46.145) (width 0.25) (layer F.Cu) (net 23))
 (via (at 68.6 43.8) (size 0.8) (drill 0.4) (layers F.Cu B.Cu) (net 23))
 (segment (start 69.385 43.015) (end 68.6 43.8) (width 0.25) (layer F.Cu) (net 23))
 (segment (start 69.385 42.9) (end 69.385 43.015) (width 0.25) (layer F.Cu) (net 23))
 (segment (start 68.999999 43.400001) (end 68.6 43.8) (width 0.25) (layer F.Cu) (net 23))
 (segment (start 69.3 43.4) (end 68.999999 43.400001) (width 0.25) (layer F.Cu) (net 23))
 (via (at 66.1 40) (size 0.8) (drill 0.4) (layers F.Cu B.Cu) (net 23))
 (segment (start 66.2 39.9) (end 66.1 40) (width 0.25) (layer F.Cu) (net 23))
 (segment (start 67.425 39.9) (end 66.2 39.9) (width 0.25) (layer F.Cu) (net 23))
 (via (at 68.8 33.4) (size 0.8) (drill 0.4) (layers F.Cu B.Cu) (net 23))
 (segment (start 69.025 33.625) (end 68.8 33.4) (width 0.25) (layer F.Cu) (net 23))
 (segment (start 69.025 34.3) (end 69.025 33.625) (width 0.25) (layer F.Cu) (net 23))
 (via (at 66.3 33.5) (size 0.8) (drill 0.4) (layers F.Cu B.Cu) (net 23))
 (segment (start 66.755 33.955) (end 66.3 33.5) (width 0.25) (layer F.Cu) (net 23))
 (segment (start 66.755 34.55) (end 66.755 33.955) (width 0.25) (layer F.Cu) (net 23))
 (segment (start 66.755 45.25) (end 69.15 45.25) (width 0.25) (layer F.Cu) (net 23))
 (segment (start 69.15 45.25) (end 69.4 45.5) (width 0.25) (layer F.Cu) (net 23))
 (segment (start 66.755 34.55) (end 69.25 34.55) (width 0.25) (layer F.Cu) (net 23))
 (segment (start 69.25 34.55) (end 69.1 34.4) (width 0.25) (layer F.Cu) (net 23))
 (segment (start 69.1 34.4) (end 67.1 34.4) (width 0.25) (layer F.Cu) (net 23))
 (segment (start 34.575 40) (end 36 40) (width 0.25) (layer F.Cu) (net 23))
 (segment (start 36 40) (end 36 40) (width 0.25) (layer F.Cu) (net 23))
 (via (at 36 40) (size 0.8) (drill 0.4) (layers F.Cu B.Cu) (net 23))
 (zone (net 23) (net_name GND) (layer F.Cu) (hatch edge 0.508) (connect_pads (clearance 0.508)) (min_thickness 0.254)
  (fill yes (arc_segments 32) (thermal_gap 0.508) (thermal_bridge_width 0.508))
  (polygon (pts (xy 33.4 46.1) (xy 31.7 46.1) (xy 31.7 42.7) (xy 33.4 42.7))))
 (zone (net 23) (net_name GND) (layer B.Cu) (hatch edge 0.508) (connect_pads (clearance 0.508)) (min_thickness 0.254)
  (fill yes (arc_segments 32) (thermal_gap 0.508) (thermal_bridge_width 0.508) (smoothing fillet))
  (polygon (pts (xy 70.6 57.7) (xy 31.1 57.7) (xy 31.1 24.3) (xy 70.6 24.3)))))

